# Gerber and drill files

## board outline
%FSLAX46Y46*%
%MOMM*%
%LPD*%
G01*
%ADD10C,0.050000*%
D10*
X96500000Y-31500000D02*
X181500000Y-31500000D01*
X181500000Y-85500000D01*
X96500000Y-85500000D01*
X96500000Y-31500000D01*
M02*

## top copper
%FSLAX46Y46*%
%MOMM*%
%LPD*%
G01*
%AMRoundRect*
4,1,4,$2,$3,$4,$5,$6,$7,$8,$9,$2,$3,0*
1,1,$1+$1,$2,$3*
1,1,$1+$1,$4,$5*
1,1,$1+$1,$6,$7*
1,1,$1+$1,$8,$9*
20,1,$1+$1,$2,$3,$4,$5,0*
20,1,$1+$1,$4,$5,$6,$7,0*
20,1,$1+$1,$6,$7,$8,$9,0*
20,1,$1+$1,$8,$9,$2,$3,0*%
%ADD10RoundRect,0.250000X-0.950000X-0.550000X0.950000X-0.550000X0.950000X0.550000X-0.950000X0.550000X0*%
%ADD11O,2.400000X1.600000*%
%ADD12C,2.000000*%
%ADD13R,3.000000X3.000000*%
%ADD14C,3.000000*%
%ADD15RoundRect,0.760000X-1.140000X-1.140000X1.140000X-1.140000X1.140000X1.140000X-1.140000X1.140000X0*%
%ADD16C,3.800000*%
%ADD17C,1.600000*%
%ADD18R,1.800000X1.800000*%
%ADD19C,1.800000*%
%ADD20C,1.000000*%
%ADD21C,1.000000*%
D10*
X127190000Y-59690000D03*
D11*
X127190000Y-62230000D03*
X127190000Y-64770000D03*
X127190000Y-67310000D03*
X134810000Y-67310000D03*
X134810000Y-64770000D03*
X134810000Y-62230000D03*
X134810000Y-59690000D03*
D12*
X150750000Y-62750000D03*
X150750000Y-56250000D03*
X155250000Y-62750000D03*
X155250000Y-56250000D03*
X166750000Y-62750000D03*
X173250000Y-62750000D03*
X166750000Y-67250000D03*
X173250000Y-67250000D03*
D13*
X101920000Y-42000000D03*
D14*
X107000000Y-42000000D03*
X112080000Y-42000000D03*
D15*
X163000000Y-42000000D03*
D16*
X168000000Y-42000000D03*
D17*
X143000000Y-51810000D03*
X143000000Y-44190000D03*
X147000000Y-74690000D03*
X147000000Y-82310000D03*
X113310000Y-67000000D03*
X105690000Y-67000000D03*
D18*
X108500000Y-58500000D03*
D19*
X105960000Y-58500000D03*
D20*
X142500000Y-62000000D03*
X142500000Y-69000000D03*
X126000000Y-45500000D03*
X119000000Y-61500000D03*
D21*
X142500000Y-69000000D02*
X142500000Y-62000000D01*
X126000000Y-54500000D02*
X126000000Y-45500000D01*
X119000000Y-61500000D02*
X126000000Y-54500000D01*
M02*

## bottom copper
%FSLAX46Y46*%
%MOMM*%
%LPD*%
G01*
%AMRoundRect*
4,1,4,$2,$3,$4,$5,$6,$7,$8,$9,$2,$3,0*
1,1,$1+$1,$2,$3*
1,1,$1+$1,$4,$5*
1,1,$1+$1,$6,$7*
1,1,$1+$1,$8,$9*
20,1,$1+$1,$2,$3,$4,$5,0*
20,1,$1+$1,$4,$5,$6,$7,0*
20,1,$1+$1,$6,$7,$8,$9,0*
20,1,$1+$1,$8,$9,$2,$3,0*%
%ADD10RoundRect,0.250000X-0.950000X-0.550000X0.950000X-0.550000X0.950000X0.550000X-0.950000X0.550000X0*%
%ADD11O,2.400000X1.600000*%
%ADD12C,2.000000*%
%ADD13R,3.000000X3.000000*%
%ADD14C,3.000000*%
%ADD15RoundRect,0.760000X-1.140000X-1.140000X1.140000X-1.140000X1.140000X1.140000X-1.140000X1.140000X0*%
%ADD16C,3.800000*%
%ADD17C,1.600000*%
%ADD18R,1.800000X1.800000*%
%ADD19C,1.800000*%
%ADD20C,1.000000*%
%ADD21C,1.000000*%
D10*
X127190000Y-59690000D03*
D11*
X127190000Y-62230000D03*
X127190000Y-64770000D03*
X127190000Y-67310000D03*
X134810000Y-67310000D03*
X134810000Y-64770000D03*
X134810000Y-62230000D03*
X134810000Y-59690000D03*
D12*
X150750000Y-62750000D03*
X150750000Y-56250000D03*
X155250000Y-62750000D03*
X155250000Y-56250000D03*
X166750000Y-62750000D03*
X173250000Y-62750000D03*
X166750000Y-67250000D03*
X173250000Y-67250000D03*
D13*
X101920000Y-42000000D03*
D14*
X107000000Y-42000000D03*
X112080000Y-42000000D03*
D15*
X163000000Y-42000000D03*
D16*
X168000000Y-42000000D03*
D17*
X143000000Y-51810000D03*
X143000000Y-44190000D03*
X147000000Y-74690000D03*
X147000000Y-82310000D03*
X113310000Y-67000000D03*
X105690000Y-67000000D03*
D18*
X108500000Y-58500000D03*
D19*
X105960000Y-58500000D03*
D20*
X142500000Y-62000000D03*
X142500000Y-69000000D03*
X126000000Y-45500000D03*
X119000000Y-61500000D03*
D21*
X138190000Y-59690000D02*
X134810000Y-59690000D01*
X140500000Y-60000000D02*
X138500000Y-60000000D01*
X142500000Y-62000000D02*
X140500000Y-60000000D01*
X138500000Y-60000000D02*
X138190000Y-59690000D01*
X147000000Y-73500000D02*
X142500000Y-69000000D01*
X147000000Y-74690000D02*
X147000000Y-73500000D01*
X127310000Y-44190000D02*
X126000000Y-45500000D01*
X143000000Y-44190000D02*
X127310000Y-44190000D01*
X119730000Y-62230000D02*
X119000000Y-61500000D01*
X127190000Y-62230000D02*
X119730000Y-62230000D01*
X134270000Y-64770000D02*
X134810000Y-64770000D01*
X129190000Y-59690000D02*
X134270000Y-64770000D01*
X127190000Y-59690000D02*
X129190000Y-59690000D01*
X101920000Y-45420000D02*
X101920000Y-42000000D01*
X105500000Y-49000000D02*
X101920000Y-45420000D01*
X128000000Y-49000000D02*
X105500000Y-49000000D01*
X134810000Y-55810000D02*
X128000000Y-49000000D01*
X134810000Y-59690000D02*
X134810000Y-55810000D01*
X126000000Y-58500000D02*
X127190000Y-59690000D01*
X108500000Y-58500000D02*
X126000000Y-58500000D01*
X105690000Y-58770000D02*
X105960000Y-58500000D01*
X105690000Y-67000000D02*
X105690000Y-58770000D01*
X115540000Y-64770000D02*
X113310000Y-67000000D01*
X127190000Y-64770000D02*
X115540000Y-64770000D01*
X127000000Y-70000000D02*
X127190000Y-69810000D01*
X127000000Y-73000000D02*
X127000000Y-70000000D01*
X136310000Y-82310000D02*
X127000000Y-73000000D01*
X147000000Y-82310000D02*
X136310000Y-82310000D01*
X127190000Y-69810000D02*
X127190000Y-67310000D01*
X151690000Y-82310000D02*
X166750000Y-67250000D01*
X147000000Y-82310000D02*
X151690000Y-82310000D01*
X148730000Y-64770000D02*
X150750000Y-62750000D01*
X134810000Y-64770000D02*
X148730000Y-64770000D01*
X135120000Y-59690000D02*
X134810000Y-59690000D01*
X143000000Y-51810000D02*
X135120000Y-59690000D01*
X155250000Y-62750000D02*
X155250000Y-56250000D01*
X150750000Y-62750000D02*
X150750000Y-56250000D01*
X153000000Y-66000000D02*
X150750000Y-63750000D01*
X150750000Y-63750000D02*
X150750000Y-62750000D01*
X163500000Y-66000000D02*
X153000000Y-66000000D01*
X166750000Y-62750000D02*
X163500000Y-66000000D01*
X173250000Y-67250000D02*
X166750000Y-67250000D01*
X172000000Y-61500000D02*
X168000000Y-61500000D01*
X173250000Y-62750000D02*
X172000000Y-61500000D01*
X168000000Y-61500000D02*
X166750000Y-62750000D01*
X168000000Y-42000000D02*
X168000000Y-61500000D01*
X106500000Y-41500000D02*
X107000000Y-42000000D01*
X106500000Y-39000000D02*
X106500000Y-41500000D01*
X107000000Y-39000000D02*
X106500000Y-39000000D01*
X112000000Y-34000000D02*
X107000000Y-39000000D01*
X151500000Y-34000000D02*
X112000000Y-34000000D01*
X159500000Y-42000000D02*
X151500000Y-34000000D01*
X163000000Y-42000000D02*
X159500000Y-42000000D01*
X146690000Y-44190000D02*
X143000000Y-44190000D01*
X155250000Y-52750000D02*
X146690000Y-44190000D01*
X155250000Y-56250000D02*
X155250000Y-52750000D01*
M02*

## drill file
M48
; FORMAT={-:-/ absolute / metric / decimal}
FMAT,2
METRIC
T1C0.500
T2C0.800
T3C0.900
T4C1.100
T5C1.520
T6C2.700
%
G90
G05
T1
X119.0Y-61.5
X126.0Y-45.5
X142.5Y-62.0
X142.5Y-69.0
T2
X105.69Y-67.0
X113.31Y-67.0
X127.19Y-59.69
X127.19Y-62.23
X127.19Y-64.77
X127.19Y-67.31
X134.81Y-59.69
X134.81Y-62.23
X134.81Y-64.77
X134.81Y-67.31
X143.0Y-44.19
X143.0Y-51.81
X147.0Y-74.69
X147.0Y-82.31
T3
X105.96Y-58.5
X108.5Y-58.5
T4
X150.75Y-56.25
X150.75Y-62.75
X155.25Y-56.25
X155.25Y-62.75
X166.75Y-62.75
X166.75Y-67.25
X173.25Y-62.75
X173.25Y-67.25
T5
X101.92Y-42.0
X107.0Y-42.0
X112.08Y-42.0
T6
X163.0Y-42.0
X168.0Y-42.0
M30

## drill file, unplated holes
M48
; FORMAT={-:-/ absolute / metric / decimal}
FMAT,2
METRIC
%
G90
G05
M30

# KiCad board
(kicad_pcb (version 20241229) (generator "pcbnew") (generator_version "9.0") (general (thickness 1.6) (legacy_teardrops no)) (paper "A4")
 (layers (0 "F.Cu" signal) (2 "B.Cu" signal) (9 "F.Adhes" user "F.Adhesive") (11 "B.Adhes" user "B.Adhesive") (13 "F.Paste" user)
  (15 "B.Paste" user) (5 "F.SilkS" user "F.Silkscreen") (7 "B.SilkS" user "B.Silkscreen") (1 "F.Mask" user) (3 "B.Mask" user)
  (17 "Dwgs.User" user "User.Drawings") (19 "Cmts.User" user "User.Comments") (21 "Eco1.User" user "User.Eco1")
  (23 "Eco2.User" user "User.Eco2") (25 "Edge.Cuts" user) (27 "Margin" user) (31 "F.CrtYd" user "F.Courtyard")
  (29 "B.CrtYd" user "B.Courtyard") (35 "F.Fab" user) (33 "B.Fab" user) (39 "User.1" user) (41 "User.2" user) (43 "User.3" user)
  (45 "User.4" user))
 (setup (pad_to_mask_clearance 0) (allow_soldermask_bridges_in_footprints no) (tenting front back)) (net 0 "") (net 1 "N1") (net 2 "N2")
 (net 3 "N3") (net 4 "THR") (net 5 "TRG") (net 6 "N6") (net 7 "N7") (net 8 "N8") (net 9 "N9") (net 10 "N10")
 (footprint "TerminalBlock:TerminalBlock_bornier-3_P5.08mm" (layer "F.Cu") (at 101.92 42)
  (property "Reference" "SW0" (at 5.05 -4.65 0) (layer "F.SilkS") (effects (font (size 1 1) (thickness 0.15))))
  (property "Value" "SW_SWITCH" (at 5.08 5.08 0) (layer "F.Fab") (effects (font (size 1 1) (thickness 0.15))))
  (pad "1" thru_hole rect (at 0 0) (size 3 3) (drill 1.52) (layers "*.Cu" "*.Mask") (remove_unused_layers no) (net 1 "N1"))
  (pad "2" thru_hole circle (at 5.08 0) (size 3 3) (drill 1.52) (layers "*.Cu" "*.Mask") (remove_unused_layers no) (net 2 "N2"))
  (pad "3" thru_hole circle (at 10.16 0) (size 3 3) (drill 1.52) (layers "*.Cu" "*.Mask") (remove_unused_layers no) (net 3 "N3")))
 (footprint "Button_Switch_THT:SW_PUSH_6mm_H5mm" (layer "F.Cu") (at 150.75 62.75 90)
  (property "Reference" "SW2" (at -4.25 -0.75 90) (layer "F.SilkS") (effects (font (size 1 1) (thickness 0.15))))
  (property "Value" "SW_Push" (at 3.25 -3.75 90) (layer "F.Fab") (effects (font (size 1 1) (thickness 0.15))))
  (pad "1" thru_hole circle (at 0 0 180) (size 2 2) (drill 1.1) (layers "*.Cu" "*.Mask") (remove_unused_layers no) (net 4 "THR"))
  (pad "1" thru_hole circle (at 6.5 0 180) (size 2 2) (drill 1.1) (layers "*.Cu" "*.Mask") (remove_unused_layers no) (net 4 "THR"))
  (pad "2" thru_hole circle (at 0 4.5 180) (size 2 2) (drill 1.1) (layers "*.Cu" "*.Mask") (remove_unused_layers no) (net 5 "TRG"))
  (pad "2" thru_hole circle (at 6.5 4.5 180) (size 2 2) (drill 1.1) (layers "*.Cu" "*.Mask") (remove_unused_layers no) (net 5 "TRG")))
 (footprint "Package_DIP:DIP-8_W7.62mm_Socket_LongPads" (layer "F.Cu") (at 127.19 59.69)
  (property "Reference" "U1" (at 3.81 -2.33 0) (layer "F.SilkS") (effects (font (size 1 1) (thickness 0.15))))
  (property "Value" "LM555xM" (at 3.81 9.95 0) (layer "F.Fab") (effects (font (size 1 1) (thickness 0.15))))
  (pad "1" thru_hole roundrect (at 0 0) (size 2.4 1.6) (drill 0.8) (layers "*.Cu" "*.Mask") (remove_unused_layers no)
   (roundrect_rratio 0.15625) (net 4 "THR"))
  (pad "2" thru_hole oval (at 0 2.54) (size 2.4 1.6) (drill 0.8) (layers "*.Cu" "*.Mask") (remove_unused_layers no) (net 5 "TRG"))
  (pad "3" thru_hole oval (at 0 5.08) (size 2.4 1.6) (drill 0.8) (layers "*.Cu" "*.Mask") (remove_unused_layers no) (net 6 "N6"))
  (pad "4" thru_hole oval (at 0 7.62) (size 2.4 1.6) (drill 0.8) (layers "*.Cu" "*.Mask") (remove_unused_layers no) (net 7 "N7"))
  (pad "5" thru_hole oval (at 7.62 7.62) (size 2.4 1.6) (drill 0.8) (layers "*.Cu" "*.Mask") (remove_unused_layers no) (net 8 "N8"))
  (pad "6" thru_hole oval (at 7.62 5.08) (size 2.4 1.6) (drill 0.8) (layers "*.Cu" "*.Mask") (remove_unused_layers no) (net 4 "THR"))
  (pad "7" thru_hole oval (at 7.62 2.54) (size 2.4 1.6) (drill 0.8) (layers "*.Cu" "*.Mask") (remove_unused_layers no) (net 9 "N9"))
  (pad "8" thru_hole oval (at 7.62 0) (size 2.4 1.6) (drill 0.8) (layers "*.Cu" "*.Mask") (remove_unused_layers no) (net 1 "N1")))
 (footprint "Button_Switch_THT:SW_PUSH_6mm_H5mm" (layer "F.Cu") (at 166.75 62.75)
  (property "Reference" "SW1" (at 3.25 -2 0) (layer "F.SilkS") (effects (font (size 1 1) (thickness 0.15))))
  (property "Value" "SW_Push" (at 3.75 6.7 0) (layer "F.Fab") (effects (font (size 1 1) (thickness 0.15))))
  (pad "1" thru_hole circle (at 0 0 90) (size 2 2) (drill 1.1) (layers "*.Cu" "*.Mask") (remove_unused_layers no) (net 4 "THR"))
  (pad "1" thru_hole circle (at 6.5 0 90) (size 2 2) (drill 1.1) (layers "*.Cu" "*.Mask") (remove_unused_layers no) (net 4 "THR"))
  (pad "2" thru_hole circle (at 0 4.5 90) (size 2 2) (drill 1.1) (layers "*.Cu" "*.Mask") (remove_unused_layers no) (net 7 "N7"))
  (pad "2" thru_hole circle (at 6.5 4.5 90) (size 2 2) (drill 1.1) (layers "*.Cu" "*.Mask") (remove_unused_layers no) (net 7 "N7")))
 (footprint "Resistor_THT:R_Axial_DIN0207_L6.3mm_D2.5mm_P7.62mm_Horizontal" (layer "F.Cu") (at 143 51.81 90)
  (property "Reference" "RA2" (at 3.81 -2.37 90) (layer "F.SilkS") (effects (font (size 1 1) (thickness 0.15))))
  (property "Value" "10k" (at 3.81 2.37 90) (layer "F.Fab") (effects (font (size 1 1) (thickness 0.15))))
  (pad "1" thru_hole circle (at 0 0 90) (size 1.6 1.6) (drill 0.8) (layers "*.Cu" "*.Mask") (remove_unused_layers no) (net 1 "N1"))
  (pad "2" thru_hole circle (at 7.62 0 90) (size 1.6 1.6) (drill 0.8) (layers "*.Cu" "*.Mask") (remove_unused_layers no) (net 5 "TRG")))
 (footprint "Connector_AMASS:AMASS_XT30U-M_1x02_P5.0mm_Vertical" (layer "F.Cu") (at 163 42)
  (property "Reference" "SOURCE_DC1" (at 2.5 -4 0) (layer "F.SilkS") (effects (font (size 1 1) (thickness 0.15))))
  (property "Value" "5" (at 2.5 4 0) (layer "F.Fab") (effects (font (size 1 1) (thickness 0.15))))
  (pad "1" thru_hole roundrect (at 0 0) (size 3.8 3.8) (drill 2.7) (layers "*.Cu" "*.Mask") (remove_unused_layers no) (roundrect_rratio 0.2)
   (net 2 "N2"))
  (pad "2" thru_hole circle (at 5 0) (size 3.8 3.8) (drill 2.7) (layers "*.Cu" "*.Mask") (remove_unused_layers no) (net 4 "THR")))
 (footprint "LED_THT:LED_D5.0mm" (layer "F.Cu") (at 108.5 58.5 180)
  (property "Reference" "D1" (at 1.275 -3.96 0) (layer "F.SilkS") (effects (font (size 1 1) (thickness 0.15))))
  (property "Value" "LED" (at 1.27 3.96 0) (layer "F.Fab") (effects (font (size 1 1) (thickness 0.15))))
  (pad "1" thru_hole rect (at 0 0 180) (size 1.8 1.8) (drill 0.9) (layers "*.Cu" "*.Mask") (remove_unused_layers no) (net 4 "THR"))
  (pad "2" thru_hole circle (at 2.54 0 180) (size 1.8 1.8) (drill 0.9) (layers "*.Cu" "*.Mask") (remove_unused_layers no) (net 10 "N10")))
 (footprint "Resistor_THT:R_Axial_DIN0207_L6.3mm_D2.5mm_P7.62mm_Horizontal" (layer "F.Cu") (at 113.31 67 180)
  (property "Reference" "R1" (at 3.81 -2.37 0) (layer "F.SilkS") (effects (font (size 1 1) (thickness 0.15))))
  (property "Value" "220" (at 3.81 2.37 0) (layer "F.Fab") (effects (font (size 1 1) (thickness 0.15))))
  (pad "1" thru_hole circle (at 0 0 180) (size 1.6 1.6) (drill 0.8) (layers "*.Cu" "*.Mask") (remove_unused_layers no) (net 6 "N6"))
  (pad "2" thru_hole circle (at 7.62 0 180) (size 1.6 1.6) (drill 0.8) (layers "*.Cu" "*.Mask") (remove_unused_layers no) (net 10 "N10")))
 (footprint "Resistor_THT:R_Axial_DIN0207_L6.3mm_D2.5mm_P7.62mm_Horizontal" (layer "F.Cu") (at 147 74.69 -90)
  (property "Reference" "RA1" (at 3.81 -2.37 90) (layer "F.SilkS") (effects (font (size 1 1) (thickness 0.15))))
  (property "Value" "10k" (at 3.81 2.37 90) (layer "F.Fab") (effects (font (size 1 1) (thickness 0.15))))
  (pad "1" thru_hole circle (at 0 0 270) (size 1.6 1.6) (drill 0.8) (layers "*.Cu" "*.Mask") (remove_unused_layers no) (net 1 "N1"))
  (pad "2" thru_hole circle (at 7.62 0 270) (size 1.6 1.6) (drill 0.8) (layers "*.Cu" "*.Mask") (remove_unused_layers no) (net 7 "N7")))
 (gr_rect (start 96.5 31.5) (end 181.5 85.5) (stroke (width 0.05) (type default)) (fill no) (layer "Edge.Cuts"))
 (segment (start 105.69 67) (end 105.69 58.77) (width 1) (layer "B.Cu") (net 10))
 (segment (start 105.69 58.77) (end 105.96 58.5) (width 1) (layer "B.Cu") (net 10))
 (segment (start 127.19 59.69) (end 129.19 59.69) (width 1) (layer "B.Cu") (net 4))
 (segment (start 168 61.5) (end 166.75 62.75) (width 1) (layer "B.Cu") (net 4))
 (segment (start 172 61.5) (end 168 61.5) (width 1) (layer "B.Cu") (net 4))
 (segment (start 108.5 58.5) (end 126 58.5) (width 1) (layer "B.Cu") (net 4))
 (segment (start 166.75 62.75) (end 163.5 66) (width 1) (layer "B.Cu") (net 4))
 (segment (start 148.73 64.77) (end 150.75 62.75) (width 1) (layer "B.Cu") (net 4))
 (segment (start 129.19 59.69) (end 134.27 64.77) (width 1) (layer "B.Cu") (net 4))
 (segment (start 134.81 64.77) (end 148.73 64.77) (width 1) (layer "B.Cu") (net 4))
 (segment (start 173.25 62.75) (end 172 61.5) (width 1) (layer "B.Cu") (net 4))
 (segment (start 153 66) (end 150.75 63.75) (width 1) (layer "B.Cu") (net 4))
 (segment (start 163.5 66) (end 153 66) (width 1) (layer "B.Cu") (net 4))
 (segment (start 134.27 64.77) (end 134.81 64.77) (width 1) (layer "B.Cu") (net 4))
 (segment (start 150.75 62.75) (end 150.75 56.25) (width 1) (layer "B.Cu") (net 4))
 (segment (start 150.75 63.75) (end 150.75 62.75) (width 1) (layer "B.Cu") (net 4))
 (segment (start 126 58.5) (end 127.19 59.69) (width 1) (layer "B.Cu") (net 4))
 (segment (start 168 42) (end 168 61.5) (width 1) (layer "B.Cu") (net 4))
 (segment (start 127.19 64.77) (end 115.54 64.77) (width 1) (layer "B.Cu") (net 6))
 (segment (start 115.54 64.77) (end 113.31 67) (width 1) (layer "B.Cu") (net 6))
 (segment (start 142.5 69) (end 142.5 62) (width 1) (layer "F.Cu") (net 1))
 (via (at 142.5 69) (size 1) (drill 0.5) (layers "F.Cu" "B.Cu") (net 1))
 (via (at 142.5 62) (size 1) (drill 0.5) (layers "F.Cu" "B.Cu") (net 1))
 (segment (start 138.19 59.69) (end 134.81 59.69) (width 1) (layer "B.Cu") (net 1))
 (segment (start 134.81 59.69) (end 134.81 55.81) (width 1) (layer "B.Cu") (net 1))
 (segment (start 140.5 60) (end 138.5 60) (width 1) (layer "B.Cu") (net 1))
 (segment (start 128 49) (end 105.5 49) (width 1) (layer "B.Cu") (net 1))
 (segment (start 147 73.5) (end 142.5 69) (width 1) (layer "B.Cu") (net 1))
 (segment (start 143 51.81) (end 135.12 59.69) (width 1) (layer "B.Cu") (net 1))
 (segment (start 138.5 60) (end 138.19 59.69) (width 1) (layer "B.Cu") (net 1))
 (segment (start 142.5 62) (end 140.5 60) (width 1) (layer "B.Cu") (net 1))
 (segment (start 147 74.69) (end 147 73.5) (width 1) (layer "B.Cu") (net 1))
 (segment (start 101.92 45.42) (end 101.92 42) (width 1) (layer "B.Cu") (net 1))
 (segment (start 105.5 49) (end 101.92 45.42) (width 1) (layer "B.Cu") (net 1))
 (segment (start 134.81 55.81) (end 128 49) (width 1) (layer "B.Cu") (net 1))
 (segment (start 135.12 59.69) (end 134.81 59.69) (width 1) (layer "B.Cu") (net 1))
 (segment (start 136.31 82.31) (end 127 73) (width 1) (layer "B.Cu") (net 7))
 (segment (start 151.69 82.31) (end 166.75 67.25) (width 1) (layer "B.Cu") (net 7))
 (segment (start 127 73) (end 127 70) (width 1) (layer "B.Cu") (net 7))
 (segment (start 147 82.31) (end 136.31 82.31) (width 1) (layer "B.Cu") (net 7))
 (segment (start 127 70) (end 127.19 69.81) (width 1) (layer "B.Cu") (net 7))
 (segment (start 147 82.31) (end 151.69 82.31) (width 1) (layer "B.Cu") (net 7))
 (segment (start 127.19 69.81) (end 127.19 67.31) (width 1) (layer "B.Cu") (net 7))
 (segment (start 173.25 67.25) (end 166.75 67.25) (width 1) (layer "B.Cu") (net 7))
 (segment (start 119 61.5) (end 126 54.5) (width 1) (layer "F.Cu") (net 5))
 (segment (start 126 54.5) (end 126 45.5) (width 1) (layer "F.Cu") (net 5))
 (via (at 119 61.5) (size 1) (drill 0.5) (layers "F.Cu" "B.Cu") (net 5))
 (via (at 126 45.5) (size 1) (drill 0.5) (layers "F.Cu" "B.Cu") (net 5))
 (segment (start 155.25 52.75) (end 146.69 44.19) (width 1) (layer "B.Cu") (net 5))
 (segment (start 155.25 62.75) (end 155.25 56.25) (width 1) (layer "B.Cu") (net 5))
 (segment (start 119.73 62.23) (end 119 61.5) (width 1) (layer "B.Cu") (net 5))
 (segment (start 155.25 56.25) (end 155.25 52.75) (width 1) (layer "B.Cu") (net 5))
 (segment (start 127.31 44.19) (end 126 45.5) (width 1) (layer "B.Cu") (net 5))
 (segment (start 143 44.19) (end 127.31 44.19) (width 1) (layer "B.Cu") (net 5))
 (segment (start 146.69 44.19) (end 143 44.19) (width 1) (layer "B.Cu") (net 5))
 (segment (start 127.19 62.23) (end 119.73 62.23) (width 1) (layer "B.Cu") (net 5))
 (segment (start 112 34) (end 107 39) (width 1) (layer "B.Cu") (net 2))
 (segment (start 163 42) (end 159.5 42) (width 1) (layer "B.Cu") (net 2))
 (segment (start 106.5 41.5) (end 107 42) (width 1) (layer "B.Cu") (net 2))
 (segment (start 106.5 39) (end 106.5 41.5) (width 1) (layer "B.Cu") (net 2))
 (segment (start 159.5 42) (end 151.5 34) (width 1) (layer "B.Cu") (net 2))
 (segment (start 151.5 34) (end 112 34) (width 1) (layer "B.Cu") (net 2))
 (segment (start 107 39) (end 106.5 39) (width 1) (layer "B.Cu") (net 2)))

